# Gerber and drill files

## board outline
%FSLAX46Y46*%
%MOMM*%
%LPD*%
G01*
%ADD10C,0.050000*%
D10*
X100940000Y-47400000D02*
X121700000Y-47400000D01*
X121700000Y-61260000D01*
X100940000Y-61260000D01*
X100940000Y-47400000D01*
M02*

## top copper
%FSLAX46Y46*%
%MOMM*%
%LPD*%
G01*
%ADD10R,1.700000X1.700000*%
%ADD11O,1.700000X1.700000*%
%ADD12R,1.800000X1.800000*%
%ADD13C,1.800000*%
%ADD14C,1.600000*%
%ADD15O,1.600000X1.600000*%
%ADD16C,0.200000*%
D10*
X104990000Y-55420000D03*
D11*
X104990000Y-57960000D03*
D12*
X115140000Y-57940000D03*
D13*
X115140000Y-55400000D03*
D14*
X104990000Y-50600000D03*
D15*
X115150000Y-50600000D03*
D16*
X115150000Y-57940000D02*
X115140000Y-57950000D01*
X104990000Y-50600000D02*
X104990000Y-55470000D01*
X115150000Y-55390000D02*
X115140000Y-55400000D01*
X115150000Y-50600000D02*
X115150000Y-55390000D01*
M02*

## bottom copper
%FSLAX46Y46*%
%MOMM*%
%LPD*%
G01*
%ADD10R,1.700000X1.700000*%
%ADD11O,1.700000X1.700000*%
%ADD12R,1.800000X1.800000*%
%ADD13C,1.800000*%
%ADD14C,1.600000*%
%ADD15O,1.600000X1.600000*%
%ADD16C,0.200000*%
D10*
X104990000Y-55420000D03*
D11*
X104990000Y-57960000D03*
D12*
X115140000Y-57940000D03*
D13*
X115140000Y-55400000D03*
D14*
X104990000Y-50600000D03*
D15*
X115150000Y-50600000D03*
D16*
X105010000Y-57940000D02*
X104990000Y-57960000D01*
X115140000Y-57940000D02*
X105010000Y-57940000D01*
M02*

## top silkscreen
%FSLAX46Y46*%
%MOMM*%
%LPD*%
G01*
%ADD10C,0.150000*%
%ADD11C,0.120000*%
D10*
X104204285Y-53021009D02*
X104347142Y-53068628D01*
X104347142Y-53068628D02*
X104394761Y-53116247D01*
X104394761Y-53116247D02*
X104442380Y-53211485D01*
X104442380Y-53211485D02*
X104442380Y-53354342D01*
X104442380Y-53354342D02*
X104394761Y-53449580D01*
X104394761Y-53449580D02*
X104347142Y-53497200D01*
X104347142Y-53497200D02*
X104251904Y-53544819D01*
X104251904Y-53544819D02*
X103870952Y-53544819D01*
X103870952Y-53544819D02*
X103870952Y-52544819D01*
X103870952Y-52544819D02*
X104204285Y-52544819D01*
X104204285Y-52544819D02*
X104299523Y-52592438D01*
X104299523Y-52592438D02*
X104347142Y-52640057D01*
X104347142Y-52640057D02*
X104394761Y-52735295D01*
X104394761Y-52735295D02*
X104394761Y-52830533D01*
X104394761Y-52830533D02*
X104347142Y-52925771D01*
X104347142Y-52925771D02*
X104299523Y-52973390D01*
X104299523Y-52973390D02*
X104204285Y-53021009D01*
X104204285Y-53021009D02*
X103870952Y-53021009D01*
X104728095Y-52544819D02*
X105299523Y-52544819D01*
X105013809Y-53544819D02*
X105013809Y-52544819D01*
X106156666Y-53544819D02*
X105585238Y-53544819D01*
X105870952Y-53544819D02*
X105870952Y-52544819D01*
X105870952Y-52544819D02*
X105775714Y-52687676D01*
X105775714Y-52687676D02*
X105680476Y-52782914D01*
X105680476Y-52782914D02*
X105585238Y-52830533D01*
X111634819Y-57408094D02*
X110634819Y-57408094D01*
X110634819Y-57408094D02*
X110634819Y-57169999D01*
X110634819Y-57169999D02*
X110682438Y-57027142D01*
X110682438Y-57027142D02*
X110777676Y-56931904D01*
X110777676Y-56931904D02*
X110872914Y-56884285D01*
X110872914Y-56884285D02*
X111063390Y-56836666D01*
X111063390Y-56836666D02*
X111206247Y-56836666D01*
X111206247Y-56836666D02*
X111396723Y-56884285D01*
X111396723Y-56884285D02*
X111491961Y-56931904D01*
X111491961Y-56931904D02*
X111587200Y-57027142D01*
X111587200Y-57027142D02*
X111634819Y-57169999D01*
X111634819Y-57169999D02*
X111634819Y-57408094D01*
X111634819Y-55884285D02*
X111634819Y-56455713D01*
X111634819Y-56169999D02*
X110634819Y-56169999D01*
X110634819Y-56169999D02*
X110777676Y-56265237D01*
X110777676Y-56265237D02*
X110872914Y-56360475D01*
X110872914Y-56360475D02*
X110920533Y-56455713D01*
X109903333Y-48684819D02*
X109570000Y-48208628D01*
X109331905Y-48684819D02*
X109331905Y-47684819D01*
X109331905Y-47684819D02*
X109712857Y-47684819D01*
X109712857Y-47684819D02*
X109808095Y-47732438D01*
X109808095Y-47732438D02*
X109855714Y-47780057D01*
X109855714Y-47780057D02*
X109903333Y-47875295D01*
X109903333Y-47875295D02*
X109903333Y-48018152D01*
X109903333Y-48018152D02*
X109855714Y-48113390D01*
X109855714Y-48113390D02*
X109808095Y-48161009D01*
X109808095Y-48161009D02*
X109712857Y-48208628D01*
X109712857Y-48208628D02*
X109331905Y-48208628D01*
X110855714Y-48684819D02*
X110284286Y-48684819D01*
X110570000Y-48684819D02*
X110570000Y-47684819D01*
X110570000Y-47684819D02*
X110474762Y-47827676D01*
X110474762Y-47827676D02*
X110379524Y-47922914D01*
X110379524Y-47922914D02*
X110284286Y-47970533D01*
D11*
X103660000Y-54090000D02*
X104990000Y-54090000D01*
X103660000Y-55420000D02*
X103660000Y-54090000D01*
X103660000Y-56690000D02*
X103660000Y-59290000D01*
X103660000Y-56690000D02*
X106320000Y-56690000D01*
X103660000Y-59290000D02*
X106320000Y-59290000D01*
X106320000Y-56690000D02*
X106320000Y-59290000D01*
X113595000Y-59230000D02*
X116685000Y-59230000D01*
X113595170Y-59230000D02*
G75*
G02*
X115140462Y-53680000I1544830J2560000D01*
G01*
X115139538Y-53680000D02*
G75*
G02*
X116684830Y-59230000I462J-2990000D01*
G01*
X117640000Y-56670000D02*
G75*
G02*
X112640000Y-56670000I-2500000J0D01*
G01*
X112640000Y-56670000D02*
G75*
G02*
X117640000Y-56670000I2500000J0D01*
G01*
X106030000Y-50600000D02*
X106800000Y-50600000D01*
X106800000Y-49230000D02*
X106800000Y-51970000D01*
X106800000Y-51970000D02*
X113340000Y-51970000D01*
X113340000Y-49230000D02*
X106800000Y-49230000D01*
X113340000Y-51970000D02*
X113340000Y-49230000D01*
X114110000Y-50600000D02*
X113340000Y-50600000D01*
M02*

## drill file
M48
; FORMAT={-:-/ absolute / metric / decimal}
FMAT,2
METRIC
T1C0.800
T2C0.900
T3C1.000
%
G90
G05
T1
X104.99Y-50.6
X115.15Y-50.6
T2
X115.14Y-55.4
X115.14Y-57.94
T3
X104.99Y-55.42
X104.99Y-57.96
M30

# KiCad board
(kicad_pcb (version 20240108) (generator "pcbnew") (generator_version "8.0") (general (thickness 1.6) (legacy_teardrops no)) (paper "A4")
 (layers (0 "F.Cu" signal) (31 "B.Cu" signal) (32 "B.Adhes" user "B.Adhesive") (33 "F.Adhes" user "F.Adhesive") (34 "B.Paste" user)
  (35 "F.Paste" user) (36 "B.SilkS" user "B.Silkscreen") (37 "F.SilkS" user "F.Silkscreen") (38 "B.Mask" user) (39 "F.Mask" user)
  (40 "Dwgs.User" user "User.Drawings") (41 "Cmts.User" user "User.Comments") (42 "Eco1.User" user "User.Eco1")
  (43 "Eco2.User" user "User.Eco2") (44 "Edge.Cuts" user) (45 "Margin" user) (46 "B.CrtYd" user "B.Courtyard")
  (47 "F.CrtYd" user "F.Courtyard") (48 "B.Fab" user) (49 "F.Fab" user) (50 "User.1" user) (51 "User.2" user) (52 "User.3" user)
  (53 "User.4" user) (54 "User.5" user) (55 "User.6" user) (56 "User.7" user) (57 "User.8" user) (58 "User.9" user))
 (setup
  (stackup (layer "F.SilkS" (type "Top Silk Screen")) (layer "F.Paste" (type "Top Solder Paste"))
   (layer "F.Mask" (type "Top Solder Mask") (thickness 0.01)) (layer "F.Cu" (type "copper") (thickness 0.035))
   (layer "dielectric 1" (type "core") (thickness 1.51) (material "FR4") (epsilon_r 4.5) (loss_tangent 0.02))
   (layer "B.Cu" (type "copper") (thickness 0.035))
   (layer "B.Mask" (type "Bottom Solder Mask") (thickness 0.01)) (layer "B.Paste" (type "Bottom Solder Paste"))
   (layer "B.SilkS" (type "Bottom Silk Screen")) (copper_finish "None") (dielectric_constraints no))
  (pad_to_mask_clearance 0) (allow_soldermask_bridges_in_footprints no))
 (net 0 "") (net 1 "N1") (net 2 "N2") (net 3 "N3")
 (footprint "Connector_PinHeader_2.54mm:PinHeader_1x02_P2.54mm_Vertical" (layer "F.Cu") (at 104.99 55.42)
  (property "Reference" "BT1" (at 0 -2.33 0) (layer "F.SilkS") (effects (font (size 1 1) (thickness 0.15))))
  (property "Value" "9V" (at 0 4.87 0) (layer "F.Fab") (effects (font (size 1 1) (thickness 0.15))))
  (fp_line (start -1.33 -1.33) (end 0 -1.33) (stroke (width 0.12) (type solid)) (layer "F.SilkS"))
  (fp_line (start -1.33 0) (end -1.33 -1.33) (stroke (width 0.12) (type solid)) (layer "F.SilkS"))
  (fp_line (start -1.33 1.27) (end -1.33 3.87) (stroke (width 0.12) (type solid)) (layer "F.SilkS"))
  (fp_line (start -1.33 1.27) (end 1.33 1.27) (stroke (width 0.12) (type solid)) (layer "F.SilkS"))
  (fp_line (start -1.33 3.87) (end 1.33 3.87) (stroke (width 0.12) (type solid)) (layer "F.SilkS"))
  (fp_line (start 1.33 1.27) (end 1.33 3.87) (stroke (width 0.12) (type solid)) (layer "F.SilkS"))
  (pad "1" thru_hole rect (at 0 0) (size 1.7 1.7) (drill 1) (layers "*.Cu" "*.Mask") (remove_unused_layers no) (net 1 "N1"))
  (pad "2" thru_hole oval (at 0 2.54) (size 1.7 1.7) (drill 1) (layers "*.Cu" "*.Mask") (remove_unused_layers no) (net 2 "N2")))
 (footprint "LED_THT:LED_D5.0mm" (layer "F.Cu") (at 115.14 57.94 90)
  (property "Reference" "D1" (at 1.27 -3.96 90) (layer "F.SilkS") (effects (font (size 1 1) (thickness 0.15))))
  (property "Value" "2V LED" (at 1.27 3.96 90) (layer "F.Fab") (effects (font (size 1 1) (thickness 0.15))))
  (fp_line (start -1.29 -1.545) (end -1.29 1.545) (stroke (width 0.12) (type solid)) (layer "F.SilkS"))
  (fp_arc (start -1.29 -1.54483) (mid 2.072002 -2.880433) (end 4.26 0.000462) (stroke (width 0.12) (type solid)) (layer "F.SilkS"))
  (fp_arc (start 4.26 -0.000462) (mid 2.072002 2.880433) (end -1.29 1.54483) (stroke (width 0.12) (type solid)) (layer "F.SilkS"))
  (fp_circle (center 1.27 0) (end 3.77 0) (stroke (width 0.12) (type solid)) (fill none) (layer "F.SilkS"))
  (pad "1" thru_hole rect (at 0 0 90) (size 1.8 1.8) (drill 0.9) (layers "*.Cu" "*.Mask") (remove_unused_layers no) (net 2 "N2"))
  (pad "2" thru_hole circle (at 2.54 0 90) (size 1.8 1.8) (drill 0.9) (layers "*.Cu" "*.Mask") (remove_unused_layers no) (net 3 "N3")))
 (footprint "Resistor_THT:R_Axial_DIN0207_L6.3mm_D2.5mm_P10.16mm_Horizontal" (layer "F.Cu") (at 104.99 50.6)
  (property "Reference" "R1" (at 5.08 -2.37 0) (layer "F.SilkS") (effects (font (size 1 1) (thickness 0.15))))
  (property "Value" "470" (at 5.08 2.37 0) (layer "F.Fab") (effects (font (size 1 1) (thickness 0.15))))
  (fp_line (start 1.04 0) (end 1.81 0) (stroke (width 0.12) (type solid)) (layer "F.SilkS"))
  (fp_line (start 1.81 -1.37) (end 1.81 1.37) (stroke (width 0.12) (type solid)) (layer "F.SilkS"))
  (fp_line (start 1.81 1.37) (end 8.35 1.37) (stroke (width 0.12) (type solid)) (layer "F.SilkS"))
  (fp_line (start 8.35 -1.37) (end 1.81 -1.37) (stroke (width 0.12) (type solid)) (layer "F.SilkS"))
  (fp_line (start 8.35 1.37) (end 8.35 -1.37) (stroke (width 0.12) (type solid)) (layer "F.SilkS"))
  (fp_line (start 9.12 0) (end 8.35 0) (stroke (width 0.12) (type solid)) (layer "F.SilkS"))
  (pad "1" thru_hole circle (at 0 0) (size 1.6 1.6) (drill 0.8) (layers "*.Cu" "*.Mask") (remove_unused_layers no) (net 1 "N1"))
  (pad "2" thru_hole oval (at 10.16 0) (size 1.6 1.6) (drill 0.8) (layers "*.Cu" "*.Mask") (remove_unused_layers no) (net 3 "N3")))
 (gr_rect (start 100.94 47.4) (end 121.7 61.26) (stroke (width 0.05) (type default)) (fill none) (layer "Edge.Cuts"))
 (segment (start 115.15 57.94) (end 115.14 57.95) (width 0.2) (layer "F.Cu") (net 2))
 (segment (start 105.01 57.94) (end 104.99 57.96) (width 0.2) (layer "B.Cu") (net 2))
 (segment (start 115.14 57.94) (end 105.01 57.94) (width 0.2) (layer "B.Cu") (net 2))
 (segment (start 104.99 50.6) (end 104.99 55.47) (width 0.2) (layer "F.Cu") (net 1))
 (segment (start 115.15 55.39) (end 115.14 55.4) (width 0.2) (layer "F.Cu") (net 3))
 (segment (start 115.15 50.6) (end 115.15 55.39) (width 0.2) (layer "F.Cu") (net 3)))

